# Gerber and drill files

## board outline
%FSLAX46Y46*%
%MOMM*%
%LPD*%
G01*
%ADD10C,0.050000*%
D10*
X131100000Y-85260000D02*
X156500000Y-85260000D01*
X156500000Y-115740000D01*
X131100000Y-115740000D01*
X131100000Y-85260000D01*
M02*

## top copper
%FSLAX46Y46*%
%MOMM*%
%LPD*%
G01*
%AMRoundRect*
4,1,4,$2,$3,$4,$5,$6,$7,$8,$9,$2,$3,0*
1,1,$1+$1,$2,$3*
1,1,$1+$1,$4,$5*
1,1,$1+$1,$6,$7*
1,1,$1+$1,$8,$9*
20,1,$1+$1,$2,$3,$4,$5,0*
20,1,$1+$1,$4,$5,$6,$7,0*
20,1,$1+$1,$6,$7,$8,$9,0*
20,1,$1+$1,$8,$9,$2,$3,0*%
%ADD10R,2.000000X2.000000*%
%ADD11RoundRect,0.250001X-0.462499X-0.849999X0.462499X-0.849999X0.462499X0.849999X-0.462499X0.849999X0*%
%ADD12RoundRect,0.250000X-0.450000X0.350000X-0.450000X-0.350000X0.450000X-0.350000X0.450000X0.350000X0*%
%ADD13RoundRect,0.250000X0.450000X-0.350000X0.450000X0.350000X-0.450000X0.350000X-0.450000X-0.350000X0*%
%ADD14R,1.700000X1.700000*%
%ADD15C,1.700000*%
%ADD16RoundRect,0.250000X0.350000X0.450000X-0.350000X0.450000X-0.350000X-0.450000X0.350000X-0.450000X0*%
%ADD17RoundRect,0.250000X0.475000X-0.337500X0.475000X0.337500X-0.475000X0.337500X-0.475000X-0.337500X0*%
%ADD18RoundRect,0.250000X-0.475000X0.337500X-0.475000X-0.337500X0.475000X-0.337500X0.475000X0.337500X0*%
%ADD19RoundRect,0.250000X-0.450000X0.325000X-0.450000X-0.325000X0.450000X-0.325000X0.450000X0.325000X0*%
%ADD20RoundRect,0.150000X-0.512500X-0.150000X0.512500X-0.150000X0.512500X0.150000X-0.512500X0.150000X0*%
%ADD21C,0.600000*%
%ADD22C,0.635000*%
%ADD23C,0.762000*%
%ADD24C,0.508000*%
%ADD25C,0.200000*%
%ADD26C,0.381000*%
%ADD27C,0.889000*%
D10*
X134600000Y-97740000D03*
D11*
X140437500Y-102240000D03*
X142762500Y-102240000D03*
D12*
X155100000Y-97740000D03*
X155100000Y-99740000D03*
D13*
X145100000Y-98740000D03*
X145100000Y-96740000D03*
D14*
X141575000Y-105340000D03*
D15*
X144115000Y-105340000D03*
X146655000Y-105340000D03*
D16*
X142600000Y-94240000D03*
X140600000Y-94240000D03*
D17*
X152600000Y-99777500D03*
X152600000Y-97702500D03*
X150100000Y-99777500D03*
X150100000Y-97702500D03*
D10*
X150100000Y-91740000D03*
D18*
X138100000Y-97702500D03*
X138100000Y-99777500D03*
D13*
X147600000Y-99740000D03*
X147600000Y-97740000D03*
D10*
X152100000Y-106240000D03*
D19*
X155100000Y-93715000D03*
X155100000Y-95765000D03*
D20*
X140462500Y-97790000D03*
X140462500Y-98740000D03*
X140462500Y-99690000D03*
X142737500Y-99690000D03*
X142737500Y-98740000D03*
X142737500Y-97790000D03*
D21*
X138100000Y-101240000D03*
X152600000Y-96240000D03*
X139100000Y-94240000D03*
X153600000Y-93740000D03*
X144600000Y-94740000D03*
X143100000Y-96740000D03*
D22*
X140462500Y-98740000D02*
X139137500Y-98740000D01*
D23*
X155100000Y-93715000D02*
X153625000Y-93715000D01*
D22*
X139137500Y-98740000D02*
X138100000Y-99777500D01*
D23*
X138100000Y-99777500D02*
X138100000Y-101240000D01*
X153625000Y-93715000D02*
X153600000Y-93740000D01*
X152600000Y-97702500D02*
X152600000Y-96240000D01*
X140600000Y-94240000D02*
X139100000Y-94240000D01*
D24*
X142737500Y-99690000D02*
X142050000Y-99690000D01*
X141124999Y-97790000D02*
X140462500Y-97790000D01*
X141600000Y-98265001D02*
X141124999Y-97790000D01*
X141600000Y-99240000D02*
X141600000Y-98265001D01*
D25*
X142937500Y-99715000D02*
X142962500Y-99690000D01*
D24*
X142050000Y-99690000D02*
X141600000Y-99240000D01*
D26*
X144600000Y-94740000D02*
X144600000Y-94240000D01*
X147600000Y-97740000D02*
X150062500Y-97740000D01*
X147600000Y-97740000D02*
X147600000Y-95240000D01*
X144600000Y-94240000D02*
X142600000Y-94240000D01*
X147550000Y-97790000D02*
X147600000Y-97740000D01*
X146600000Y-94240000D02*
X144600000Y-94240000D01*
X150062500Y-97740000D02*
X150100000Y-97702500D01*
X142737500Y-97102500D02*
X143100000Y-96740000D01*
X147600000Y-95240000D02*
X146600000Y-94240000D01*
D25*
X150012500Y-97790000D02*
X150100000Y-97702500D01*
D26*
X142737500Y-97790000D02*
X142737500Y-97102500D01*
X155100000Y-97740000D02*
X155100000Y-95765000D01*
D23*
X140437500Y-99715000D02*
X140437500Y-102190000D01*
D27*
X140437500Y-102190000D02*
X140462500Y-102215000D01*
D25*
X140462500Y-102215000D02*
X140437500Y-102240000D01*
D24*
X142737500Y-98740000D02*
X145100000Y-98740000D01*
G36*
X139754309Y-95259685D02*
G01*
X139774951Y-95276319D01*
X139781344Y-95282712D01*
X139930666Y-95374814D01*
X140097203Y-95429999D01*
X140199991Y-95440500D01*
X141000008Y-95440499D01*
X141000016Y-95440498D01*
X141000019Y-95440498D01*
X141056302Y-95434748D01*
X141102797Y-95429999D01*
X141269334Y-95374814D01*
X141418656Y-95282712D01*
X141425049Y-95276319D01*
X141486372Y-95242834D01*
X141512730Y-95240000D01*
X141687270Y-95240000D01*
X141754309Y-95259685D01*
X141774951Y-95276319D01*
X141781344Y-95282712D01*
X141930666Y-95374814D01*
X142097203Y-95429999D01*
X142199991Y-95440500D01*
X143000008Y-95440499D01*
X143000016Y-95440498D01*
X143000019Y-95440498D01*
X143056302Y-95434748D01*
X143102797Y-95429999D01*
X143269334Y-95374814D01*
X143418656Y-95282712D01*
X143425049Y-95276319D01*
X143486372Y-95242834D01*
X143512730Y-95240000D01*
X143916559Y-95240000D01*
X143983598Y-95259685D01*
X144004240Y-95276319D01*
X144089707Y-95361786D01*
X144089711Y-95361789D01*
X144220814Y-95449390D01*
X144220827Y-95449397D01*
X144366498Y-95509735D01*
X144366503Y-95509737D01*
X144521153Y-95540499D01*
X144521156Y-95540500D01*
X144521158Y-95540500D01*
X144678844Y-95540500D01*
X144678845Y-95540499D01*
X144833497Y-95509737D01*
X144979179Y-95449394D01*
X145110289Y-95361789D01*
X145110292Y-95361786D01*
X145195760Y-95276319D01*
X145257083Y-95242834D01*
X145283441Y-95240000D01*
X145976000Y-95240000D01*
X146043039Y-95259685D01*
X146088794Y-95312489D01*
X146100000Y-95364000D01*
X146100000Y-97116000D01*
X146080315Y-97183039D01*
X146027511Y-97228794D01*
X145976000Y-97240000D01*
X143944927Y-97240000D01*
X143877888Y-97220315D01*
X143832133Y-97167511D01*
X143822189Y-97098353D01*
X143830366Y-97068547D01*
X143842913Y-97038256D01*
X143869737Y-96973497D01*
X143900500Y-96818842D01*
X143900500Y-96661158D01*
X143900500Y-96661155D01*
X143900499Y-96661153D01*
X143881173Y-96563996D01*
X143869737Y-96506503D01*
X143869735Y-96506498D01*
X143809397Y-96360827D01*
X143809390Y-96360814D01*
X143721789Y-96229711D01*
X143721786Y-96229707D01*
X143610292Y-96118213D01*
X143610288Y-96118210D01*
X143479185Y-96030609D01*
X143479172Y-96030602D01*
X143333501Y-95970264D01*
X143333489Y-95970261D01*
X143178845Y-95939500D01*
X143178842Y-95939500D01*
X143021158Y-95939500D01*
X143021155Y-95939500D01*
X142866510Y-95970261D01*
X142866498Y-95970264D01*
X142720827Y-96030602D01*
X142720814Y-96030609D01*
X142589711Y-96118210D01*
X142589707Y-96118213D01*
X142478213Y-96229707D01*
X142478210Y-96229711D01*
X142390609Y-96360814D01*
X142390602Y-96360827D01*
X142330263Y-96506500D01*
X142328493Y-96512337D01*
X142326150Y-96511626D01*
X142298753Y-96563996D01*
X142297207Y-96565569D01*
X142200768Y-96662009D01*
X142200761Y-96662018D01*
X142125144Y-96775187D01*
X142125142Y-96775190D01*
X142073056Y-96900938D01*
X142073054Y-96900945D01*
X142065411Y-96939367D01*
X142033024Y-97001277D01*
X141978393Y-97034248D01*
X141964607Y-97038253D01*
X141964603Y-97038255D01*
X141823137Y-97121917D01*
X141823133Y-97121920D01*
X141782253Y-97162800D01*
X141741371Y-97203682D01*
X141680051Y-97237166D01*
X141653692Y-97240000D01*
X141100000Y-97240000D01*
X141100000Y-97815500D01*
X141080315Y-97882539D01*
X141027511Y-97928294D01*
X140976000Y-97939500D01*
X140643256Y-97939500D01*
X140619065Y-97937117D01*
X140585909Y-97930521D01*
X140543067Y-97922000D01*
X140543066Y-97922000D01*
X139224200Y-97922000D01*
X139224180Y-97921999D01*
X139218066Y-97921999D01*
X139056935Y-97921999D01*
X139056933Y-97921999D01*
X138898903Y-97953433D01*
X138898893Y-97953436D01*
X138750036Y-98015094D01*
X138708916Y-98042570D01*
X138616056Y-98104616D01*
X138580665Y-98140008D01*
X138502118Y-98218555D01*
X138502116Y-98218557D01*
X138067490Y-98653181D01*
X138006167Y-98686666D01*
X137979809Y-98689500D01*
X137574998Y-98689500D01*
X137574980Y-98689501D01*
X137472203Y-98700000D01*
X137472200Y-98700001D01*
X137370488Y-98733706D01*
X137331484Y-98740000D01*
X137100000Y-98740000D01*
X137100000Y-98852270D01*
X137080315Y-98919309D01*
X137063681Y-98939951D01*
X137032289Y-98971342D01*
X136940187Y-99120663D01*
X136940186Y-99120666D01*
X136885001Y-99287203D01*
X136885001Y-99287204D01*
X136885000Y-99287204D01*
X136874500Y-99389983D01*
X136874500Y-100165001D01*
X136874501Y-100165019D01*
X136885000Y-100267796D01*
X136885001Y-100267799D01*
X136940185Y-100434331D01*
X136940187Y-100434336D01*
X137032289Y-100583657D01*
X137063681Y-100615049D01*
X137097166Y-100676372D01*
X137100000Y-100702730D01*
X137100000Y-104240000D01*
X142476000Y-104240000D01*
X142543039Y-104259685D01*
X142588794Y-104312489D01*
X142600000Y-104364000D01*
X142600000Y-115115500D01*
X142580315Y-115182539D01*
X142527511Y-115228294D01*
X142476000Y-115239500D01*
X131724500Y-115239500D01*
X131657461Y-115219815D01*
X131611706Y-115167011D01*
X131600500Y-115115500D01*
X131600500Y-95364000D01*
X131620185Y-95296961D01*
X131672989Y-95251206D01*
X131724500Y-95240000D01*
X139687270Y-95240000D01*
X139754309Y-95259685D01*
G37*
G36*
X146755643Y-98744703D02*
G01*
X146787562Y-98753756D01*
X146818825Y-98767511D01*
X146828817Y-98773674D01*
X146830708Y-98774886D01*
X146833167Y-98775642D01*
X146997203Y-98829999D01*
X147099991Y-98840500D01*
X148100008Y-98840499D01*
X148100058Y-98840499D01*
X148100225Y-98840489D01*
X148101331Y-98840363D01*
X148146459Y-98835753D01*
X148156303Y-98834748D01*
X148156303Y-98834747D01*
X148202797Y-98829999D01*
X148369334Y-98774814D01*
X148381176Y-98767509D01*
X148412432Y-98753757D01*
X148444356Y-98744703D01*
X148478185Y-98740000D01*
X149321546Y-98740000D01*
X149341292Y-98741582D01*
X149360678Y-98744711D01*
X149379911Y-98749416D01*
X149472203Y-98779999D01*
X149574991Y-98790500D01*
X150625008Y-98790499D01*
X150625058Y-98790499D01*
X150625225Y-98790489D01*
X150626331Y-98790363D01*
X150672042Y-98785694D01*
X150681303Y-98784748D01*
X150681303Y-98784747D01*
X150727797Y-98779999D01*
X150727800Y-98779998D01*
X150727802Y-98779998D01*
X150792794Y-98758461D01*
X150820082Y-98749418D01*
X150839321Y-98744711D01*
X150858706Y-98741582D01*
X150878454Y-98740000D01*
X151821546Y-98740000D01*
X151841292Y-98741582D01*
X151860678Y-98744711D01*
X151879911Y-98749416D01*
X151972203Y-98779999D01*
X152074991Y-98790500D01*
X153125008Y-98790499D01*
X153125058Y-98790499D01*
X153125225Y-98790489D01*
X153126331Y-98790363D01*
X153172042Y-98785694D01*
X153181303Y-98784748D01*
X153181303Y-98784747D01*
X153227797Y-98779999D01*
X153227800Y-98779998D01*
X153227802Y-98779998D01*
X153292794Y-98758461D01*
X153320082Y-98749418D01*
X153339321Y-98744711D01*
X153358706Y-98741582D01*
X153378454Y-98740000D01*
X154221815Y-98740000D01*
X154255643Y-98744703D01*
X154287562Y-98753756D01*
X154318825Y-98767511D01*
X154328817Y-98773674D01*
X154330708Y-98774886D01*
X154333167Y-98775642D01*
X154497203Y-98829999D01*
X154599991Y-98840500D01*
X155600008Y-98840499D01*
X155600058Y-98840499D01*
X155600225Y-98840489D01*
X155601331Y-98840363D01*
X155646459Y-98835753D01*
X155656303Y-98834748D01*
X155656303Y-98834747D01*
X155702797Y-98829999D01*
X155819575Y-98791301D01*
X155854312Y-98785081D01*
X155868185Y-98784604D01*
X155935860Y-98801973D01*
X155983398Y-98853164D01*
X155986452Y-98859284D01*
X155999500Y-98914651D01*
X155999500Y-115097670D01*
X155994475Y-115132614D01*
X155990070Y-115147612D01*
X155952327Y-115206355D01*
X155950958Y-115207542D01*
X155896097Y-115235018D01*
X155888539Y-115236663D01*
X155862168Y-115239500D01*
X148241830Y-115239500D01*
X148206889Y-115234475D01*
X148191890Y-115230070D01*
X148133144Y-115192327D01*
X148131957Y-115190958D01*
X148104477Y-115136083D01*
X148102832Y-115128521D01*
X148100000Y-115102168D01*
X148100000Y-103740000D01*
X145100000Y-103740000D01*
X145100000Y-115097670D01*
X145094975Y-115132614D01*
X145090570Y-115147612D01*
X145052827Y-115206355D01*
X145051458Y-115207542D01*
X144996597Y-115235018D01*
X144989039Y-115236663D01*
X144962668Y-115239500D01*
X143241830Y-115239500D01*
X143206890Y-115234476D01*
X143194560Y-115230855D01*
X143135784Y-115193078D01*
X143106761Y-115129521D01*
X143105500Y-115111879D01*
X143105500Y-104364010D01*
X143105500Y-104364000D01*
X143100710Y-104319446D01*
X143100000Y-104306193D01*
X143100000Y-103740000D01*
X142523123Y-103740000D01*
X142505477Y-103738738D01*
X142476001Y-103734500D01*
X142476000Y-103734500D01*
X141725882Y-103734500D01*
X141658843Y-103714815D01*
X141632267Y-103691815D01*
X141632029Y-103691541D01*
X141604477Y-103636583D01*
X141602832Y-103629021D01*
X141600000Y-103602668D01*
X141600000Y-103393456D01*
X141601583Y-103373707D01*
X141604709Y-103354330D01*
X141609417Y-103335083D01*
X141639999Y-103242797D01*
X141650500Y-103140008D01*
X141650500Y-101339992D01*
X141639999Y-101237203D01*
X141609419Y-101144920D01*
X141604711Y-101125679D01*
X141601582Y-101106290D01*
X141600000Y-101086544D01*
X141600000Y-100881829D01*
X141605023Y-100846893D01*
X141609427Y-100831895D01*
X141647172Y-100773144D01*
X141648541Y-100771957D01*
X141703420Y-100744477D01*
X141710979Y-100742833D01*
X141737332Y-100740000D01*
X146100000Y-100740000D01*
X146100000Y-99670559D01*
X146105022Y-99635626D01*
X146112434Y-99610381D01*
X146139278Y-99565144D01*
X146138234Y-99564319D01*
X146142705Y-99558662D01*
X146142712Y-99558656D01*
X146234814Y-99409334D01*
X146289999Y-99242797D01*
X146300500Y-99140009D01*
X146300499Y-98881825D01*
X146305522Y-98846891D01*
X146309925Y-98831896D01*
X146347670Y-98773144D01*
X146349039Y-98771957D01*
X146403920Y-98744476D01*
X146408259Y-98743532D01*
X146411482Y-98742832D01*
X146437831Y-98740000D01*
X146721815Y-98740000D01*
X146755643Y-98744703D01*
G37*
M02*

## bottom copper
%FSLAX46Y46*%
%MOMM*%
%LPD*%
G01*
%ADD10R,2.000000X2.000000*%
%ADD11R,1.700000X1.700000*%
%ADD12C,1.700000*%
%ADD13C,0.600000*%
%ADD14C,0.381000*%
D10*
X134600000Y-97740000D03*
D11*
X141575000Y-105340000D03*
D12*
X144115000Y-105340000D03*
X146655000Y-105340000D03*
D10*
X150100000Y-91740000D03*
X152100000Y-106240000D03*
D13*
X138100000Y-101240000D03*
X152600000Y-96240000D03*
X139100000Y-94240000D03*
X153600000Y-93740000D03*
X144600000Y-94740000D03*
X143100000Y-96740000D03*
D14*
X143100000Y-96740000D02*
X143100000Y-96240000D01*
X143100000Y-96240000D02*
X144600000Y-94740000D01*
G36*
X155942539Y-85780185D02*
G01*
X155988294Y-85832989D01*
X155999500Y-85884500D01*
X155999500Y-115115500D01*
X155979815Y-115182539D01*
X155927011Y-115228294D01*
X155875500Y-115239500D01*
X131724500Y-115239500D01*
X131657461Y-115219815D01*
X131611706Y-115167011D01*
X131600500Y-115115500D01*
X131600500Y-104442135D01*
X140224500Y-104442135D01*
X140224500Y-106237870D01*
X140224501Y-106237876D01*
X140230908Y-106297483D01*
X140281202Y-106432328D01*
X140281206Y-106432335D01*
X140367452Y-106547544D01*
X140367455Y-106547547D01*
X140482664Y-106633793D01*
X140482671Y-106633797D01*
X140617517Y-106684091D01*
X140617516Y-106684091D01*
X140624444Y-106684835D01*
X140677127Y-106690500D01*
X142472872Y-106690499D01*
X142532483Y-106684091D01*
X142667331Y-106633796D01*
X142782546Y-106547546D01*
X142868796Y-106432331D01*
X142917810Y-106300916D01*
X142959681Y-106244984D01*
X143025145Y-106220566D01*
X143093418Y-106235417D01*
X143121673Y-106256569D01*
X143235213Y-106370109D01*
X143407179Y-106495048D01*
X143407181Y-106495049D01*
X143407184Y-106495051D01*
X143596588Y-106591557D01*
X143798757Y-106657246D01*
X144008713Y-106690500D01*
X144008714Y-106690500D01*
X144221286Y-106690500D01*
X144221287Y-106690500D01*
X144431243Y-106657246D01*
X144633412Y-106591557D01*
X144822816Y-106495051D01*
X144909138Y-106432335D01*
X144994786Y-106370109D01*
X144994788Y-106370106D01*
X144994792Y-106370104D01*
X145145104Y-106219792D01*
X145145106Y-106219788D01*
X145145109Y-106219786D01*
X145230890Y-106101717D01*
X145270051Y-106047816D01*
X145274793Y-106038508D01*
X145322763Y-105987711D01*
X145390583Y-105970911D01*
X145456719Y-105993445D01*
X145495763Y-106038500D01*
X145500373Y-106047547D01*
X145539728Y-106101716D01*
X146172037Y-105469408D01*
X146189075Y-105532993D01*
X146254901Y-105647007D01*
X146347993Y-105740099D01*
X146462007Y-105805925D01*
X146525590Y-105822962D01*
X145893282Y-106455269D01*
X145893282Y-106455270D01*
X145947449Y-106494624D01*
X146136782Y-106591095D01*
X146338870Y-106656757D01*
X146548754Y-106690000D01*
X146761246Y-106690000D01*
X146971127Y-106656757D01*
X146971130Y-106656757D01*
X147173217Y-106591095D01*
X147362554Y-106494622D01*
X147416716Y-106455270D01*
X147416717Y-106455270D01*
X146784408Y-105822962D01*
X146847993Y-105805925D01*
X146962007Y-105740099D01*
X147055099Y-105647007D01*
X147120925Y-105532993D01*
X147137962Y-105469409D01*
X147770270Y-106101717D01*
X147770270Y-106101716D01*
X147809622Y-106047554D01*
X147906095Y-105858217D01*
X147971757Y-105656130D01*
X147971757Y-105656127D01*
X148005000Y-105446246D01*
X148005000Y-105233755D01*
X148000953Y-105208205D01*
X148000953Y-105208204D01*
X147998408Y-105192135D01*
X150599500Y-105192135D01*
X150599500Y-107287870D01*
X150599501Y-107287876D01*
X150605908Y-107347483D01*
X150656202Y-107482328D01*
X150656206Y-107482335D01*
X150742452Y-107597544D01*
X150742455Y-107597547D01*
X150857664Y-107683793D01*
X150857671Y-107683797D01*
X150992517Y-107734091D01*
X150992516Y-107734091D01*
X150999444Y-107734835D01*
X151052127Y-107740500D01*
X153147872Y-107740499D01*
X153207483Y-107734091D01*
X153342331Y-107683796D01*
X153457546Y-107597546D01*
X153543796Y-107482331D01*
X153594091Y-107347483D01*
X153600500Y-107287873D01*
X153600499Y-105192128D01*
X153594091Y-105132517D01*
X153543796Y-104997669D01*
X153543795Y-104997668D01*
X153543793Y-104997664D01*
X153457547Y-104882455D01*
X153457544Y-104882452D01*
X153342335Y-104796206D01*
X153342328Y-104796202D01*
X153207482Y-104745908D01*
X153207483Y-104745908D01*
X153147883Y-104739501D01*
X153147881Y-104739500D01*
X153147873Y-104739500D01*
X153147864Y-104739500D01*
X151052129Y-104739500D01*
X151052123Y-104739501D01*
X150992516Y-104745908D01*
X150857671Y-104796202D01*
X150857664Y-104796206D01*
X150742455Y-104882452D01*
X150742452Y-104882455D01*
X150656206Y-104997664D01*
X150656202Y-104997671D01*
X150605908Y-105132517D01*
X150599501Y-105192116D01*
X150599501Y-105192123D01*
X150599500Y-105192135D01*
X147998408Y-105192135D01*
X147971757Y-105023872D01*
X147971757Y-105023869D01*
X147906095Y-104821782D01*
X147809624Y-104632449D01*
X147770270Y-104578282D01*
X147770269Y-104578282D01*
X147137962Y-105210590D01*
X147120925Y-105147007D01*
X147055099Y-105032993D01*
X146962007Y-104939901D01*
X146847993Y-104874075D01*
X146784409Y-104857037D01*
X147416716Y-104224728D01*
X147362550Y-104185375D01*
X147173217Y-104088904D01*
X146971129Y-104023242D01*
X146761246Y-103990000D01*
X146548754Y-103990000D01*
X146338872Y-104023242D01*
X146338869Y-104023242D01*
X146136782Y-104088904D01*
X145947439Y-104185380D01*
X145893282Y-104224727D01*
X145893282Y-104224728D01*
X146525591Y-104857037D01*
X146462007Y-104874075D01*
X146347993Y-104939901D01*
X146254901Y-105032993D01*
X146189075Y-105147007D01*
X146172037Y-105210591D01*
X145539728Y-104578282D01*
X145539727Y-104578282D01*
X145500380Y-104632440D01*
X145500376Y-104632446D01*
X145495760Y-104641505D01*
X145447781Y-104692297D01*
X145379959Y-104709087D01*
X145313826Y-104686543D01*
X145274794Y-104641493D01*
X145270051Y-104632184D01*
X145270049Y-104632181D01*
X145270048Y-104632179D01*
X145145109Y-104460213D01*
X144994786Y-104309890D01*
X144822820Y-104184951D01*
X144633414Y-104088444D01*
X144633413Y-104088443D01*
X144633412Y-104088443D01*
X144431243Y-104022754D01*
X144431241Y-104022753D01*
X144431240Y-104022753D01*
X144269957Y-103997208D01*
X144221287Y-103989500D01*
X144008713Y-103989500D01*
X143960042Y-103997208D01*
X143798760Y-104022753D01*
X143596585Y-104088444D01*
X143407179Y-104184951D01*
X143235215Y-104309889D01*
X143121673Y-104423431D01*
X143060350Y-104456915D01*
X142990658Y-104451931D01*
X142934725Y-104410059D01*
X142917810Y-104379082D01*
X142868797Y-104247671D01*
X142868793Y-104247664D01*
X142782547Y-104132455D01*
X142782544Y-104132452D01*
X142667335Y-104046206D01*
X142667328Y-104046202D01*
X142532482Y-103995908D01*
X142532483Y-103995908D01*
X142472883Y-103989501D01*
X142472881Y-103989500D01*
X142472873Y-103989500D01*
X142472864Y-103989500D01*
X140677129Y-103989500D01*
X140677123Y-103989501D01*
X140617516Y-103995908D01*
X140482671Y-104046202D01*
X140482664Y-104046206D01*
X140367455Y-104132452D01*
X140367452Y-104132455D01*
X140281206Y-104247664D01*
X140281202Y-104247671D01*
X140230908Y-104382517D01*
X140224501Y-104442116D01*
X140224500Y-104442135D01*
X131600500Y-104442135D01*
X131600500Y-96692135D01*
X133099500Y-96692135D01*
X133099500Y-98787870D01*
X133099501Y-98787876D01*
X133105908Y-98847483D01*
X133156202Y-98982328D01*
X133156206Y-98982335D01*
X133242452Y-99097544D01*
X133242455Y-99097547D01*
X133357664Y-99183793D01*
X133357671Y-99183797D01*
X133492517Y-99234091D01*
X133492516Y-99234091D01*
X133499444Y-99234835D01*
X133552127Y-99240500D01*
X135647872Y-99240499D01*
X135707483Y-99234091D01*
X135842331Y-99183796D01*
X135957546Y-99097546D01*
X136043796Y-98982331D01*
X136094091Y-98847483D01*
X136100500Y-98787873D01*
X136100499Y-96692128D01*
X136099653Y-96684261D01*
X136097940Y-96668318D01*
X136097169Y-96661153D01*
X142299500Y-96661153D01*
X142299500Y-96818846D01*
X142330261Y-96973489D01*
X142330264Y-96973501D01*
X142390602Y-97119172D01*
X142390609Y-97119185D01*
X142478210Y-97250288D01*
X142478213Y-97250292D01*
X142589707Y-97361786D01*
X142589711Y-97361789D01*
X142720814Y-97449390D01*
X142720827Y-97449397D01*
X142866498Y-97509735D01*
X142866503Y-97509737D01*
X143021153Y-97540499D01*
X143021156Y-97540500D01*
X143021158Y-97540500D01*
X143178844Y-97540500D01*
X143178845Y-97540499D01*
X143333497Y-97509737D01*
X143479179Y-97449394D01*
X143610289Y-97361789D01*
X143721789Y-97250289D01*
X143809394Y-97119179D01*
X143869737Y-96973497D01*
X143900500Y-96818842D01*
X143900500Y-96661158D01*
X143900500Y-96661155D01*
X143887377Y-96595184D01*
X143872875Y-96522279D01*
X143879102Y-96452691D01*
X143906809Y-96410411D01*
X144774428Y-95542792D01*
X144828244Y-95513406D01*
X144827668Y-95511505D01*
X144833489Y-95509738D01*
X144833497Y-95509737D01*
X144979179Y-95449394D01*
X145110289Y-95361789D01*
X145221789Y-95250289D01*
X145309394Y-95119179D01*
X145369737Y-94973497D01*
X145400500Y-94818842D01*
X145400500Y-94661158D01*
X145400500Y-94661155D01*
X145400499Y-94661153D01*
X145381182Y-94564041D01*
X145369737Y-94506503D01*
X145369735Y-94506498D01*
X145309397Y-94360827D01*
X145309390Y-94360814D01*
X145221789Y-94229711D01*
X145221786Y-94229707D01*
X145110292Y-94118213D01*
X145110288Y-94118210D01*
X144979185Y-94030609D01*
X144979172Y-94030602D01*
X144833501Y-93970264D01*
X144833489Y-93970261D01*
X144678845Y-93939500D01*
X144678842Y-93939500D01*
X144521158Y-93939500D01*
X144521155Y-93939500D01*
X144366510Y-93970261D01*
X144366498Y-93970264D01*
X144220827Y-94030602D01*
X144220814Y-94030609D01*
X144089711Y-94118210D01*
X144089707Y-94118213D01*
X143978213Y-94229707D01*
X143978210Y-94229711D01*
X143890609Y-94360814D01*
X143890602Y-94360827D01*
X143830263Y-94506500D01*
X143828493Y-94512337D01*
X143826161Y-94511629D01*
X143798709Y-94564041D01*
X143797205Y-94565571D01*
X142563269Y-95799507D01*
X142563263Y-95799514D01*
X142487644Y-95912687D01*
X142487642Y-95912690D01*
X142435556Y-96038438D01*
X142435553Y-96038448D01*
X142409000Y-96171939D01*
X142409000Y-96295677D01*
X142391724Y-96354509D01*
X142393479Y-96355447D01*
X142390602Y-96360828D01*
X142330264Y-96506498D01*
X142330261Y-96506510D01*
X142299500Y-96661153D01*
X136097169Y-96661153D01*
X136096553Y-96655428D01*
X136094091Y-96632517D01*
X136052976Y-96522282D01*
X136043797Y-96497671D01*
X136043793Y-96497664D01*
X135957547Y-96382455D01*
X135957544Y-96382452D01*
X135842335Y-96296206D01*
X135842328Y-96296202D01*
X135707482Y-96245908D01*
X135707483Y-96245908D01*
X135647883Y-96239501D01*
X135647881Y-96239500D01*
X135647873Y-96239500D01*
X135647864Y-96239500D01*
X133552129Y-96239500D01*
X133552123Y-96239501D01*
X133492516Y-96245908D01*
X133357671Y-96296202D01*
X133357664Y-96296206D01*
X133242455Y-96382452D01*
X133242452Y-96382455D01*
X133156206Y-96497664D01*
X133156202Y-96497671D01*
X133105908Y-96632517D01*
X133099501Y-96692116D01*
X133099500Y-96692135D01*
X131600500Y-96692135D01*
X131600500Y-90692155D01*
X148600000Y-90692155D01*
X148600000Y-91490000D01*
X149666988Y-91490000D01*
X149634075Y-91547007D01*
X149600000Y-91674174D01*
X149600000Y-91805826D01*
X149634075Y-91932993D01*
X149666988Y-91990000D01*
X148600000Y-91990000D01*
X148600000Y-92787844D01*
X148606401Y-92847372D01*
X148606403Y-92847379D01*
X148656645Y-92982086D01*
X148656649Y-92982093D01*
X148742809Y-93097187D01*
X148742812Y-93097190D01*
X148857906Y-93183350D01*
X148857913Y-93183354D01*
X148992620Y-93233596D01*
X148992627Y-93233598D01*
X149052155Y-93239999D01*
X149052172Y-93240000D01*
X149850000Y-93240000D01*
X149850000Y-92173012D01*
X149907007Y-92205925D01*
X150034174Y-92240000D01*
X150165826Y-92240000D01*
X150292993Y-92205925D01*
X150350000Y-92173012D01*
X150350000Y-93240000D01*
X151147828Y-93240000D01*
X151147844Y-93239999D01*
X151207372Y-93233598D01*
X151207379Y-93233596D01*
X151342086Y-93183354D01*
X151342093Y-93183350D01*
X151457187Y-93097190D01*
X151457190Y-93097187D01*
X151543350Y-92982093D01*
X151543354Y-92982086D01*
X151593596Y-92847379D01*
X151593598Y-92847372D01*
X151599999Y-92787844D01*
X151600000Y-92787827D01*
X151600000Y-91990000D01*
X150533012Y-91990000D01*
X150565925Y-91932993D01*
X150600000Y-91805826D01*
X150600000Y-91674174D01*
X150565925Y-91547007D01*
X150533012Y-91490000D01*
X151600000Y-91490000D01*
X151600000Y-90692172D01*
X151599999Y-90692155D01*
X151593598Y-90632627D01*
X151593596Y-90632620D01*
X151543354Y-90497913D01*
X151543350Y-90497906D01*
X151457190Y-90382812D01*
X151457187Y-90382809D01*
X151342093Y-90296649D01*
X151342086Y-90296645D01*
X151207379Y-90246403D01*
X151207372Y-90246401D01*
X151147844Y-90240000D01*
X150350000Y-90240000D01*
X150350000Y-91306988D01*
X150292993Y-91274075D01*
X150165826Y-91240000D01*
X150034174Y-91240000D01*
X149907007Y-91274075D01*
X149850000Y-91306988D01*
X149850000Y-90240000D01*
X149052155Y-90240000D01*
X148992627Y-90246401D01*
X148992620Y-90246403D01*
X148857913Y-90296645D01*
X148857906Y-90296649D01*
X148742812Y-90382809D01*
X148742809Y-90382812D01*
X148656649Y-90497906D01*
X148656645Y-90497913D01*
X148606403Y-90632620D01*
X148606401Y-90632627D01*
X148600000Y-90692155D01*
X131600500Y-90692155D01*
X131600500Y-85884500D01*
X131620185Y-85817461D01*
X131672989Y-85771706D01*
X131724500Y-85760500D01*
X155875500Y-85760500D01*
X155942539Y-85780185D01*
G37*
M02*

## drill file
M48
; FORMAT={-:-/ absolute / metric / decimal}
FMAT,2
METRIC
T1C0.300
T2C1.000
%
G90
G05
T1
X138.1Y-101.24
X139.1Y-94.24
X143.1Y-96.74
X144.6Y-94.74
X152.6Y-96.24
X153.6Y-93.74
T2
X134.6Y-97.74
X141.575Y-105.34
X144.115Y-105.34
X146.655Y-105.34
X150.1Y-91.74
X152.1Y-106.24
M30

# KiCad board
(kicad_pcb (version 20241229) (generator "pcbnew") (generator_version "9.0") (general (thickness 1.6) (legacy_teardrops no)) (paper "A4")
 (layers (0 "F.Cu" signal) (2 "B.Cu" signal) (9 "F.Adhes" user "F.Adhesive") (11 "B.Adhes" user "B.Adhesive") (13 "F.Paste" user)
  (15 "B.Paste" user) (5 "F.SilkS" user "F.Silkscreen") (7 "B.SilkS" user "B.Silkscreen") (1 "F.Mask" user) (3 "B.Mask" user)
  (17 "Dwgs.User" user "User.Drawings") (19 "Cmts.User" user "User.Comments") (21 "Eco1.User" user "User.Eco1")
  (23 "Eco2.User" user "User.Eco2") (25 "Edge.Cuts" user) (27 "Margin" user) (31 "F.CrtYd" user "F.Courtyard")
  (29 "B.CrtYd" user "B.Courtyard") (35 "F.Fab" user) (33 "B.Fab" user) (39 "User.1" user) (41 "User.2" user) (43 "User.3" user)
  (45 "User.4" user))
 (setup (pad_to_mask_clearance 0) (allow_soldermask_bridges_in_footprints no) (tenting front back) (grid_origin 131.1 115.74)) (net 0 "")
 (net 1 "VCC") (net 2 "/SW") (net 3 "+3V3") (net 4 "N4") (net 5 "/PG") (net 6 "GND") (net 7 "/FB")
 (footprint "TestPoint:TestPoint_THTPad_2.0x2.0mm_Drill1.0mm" (layer "F.Cu") (at 134.6 97.74)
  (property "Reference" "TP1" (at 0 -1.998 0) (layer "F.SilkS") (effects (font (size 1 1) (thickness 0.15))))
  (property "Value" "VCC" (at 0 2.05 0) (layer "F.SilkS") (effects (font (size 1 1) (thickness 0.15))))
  (pad "1" thru_hole rect (at 0 0) (size 2 2) (drill 1) (layers "*.Cu" "*.Mask") (remove_unused_layers no) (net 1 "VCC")))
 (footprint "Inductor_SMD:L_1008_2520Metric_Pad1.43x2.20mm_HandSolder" (layer "F.Cu") (at 141.6 102.24)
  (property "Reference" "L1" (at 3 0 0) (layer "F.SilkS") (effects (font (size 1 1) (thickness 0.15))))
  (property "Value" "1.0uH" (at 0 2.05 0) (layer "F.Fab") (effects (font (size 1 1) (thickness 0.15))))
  (pad "1" smd roundrect (at -1.1625 0) (size 1.425 2.2) (layers "F.Cu" "F.Mask" "F.Paste") (roundrect_rratio 0.175439) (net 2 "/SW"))
  (pad "2" smd roundrect (at 1.1625 0) (size 1.425 2.2) (layers "F.Cu" "F.Mask" "F.Paste") (roundrect_rratio 0.175439) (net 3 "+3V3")))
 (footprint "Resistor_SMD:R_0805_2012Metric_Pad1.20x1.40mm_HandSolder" (layer "F.Cu") (at 155.1 98.74 -90)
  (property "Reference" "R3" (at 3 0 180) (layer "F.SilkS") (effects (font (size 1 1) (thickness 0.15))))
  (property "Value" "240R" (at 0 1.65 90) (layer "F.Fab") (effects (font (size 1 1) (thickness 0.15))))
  (pad "1" smd roundrect (at -1 0 270) (size 1.2 1.4) (layers "F.Cu" "F.Mask" "F.Paste") (roundrect_rratio 0.208333) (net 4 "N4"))
  (pad "2" smd roundrect (at 1 0 270) (size 1.2 1.4) (layers "F.Cu" "F.Mask" "F.Paste") (roundrect_rratio 0.208333) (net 3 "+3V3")))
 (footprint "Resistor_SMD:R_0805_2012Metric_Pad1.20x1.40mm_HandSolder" (layer "F.Cu") (at 145.1 97.74 90)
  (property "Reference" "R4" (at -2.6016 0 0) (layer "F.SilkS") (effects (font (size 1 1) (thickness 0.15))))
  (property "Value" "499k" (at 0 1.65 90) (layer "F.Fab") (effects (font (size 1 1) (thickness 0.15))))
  (pad "1" smd roundrect (at -1 0 90) (size 1.2 1.4) (layers "F.Cu" "F.Mask" "F.Paste") (roundrect_rratio 0.208333) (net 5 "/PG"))
  (pad "2" smd roundrect (at 1 0 90) (size 1.2 1.4) (layers "F.Cu" "F.Mask" "F.Paste") (roundrect_rratio 0.208333) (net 1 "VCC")))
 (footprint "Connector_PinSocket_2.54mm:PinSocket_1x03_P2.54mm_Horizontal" (layer "F.Cu") (at 141.575 105.34 90)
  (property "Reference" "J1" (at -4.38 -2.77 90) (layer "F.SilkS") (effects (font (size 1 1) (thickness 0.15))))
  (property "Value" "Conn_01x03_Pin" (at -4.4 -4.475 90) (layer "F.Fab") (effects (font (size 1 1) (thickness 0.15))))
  (pad "1" thru_hole rect (at 0 0 90) (size 1.7 1.7) (drill 1) (layers "*.Cu" "*.Mask") (remove_unused_layers no) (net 1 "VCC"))
  (pad "2" thru_hole circle (at 0 2.54 90) (size 1.7 1.7) (drill 1) (layers "*.Cu" "*.Mask") (remove_unused_layers no) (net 3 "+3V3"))
  (pad "3" thru_hole circle (at 0 5.08 90) (size 1.7 1.7) (drill 1) (layers "*.Cu" "*.Mask") (remove_unused_layers no) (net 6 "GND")))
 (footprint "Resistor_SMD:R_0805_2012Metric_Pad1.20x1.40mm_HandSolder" (layer "F.Cu") (at 141.6 94.24 180)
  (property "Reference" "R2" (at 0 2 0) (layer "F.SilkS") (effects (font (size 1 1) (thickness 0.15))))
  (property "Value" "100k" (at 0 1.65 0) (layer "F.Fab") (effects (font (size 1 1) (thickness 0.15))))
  (pad "1" smd roundrect (at -1 0 180) (size 1.2 1.4) (layers "F.Cu" "F.Mask" "F.Paste") (roundrect_rratio 0.208333) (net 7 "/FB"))
  (pad "2" smd roundrect (at 1 0 180) (size 1.2 1.4) (layers "F.Cu" "F.Mask" "F.Paste") (roundrect_rratio 0.208333) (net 6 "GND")))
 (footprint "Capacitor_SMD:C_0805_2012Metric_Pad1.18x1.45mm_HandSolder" (layer "F.Cu") (at 152.6 98.74 90)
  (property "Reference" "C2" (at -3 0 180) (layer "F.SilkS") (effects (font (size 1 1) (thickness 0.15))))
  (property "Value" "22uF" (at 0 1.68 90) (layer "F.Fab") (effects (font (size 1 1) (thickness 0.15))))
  (pad "1" smd roundrect (at -1.0375 0 90) (size 1.175 1.45) (layers "F.Cu" "F.Mask" "F.Paste") (roundrect_rratio 0.212766) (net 3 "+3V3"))
  (pad "2" smd roundrect (at 1.0375 0 90) (size 1.175 1.45) (layers "F.Cu" "F.Mask" "F.Paste") (roundrect_rratio 0.212766) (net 6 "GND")))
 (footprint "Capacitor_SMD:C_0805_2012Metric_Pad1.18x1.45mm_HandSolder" (layer "F.Cu") (at 150.1 98.74 90)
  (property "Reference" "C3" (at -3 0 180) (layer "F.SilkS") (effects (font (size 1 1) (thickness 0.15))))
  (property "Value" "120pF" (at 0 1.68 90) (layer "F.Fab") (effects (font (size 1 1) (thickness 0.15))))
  (pad "1" smd roundrect (at -1.0375 0 90) (size 1.175 1.45) (layers "F.Cu" "F.Mask" "F.Paste") (roundrect_rratio 0.212766) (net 3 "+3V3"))
  (pad "2" smd roundrect (at 1.0375 0 90) (size 1.175 1.45) (layers "F.Cu" "F.Mask" "F.Paste") (roundrect_rratio 0.212766) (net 7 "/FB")))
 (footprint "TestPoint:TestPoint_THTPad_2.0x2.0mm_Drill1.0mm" (layer "F.Cu") (at 150.1 91.74)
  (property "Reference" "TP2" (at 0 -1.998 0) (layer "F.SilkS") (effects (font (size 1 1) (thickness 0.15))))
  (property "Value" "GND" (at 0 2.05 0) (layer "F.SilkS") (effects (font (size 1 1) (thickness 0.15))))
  (pad "1" thru_hole rect (at 0 0) (size 2 2) (drill 1) (layers "*.Cu" "*.Mask") (remove_unused_layers no) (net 6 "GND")))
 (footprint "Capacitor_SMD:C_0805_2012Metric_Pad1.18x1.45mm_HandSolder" (layer "F.Cu") (at 138.1 98.74 -90)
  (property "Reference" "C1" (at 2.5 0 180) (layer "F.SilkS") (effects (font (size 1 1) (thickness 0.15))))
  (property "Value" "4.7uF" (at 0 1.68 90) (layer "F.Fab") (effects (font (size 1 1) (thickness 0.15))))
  (pad "1" smd roundrect (at -1.0375 0 270) (size 1.175 1.45) (layers "F.Cu" "F.Mask" "F.Paste") (roundrect_rratio 0.212766) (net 1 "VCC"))
  (pad "2" smd roundrect (at 1.0375 0 270) (size 1.175 1.45) (layers "F.Cu" "F.Mask" "F.Paste") (roundrect_rratio 0.212766) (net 6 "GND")))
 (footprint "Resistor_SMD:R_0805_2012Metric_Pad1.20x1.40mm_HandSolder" (layer "F.Cu") (at 147.6 98.74 90)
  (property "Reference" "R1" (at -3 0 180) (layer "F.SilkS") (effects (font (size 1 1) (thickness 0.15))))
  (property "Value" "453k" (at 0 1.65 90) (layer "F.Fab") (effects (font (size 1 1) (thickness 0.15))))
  (pad "1" smd roundrect (at -1 0 90) (size 1.2 1.4) (layers "F.Cu" "F.Mask" "F.Paste") (roundrect_rratio 0.208333) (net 3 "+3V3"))
  (pad "2" smd roundrect (at 1 0 90) (size 1.2 1.4) (layers "F.Cu" "F.Mask" "F.Paste") (roundrect_rratio 0.208333) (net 7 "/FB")))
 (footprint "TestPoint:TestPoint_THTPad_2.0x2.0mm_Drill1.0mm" (layer "F.Cu") (at 152.1 106.24)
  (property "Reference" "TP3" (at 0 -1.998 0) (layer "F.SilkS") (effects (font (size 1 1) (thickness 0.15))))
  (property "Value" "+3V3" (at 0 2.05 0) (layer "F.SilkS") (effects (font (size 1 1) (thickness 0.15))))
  (pad "1" thru_hole rect (at 0 0) (size 2 2) (drill 1) (layers "*.Cu" "*.Mask") (remove_unused_layers no) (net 3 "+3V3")))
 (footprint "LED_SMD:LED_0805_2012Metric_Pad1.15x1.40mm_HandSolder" (layer "F.Cu") (at 155.1 94.74 -90)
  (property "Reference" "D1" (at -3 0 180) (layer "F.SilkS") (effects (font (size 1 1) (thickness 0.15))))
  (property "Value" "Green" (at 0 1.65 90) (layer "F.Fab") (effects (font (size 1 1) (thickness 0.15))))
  (pad "1" smd roundrect (at -1.025 0 270) (size 1.15 1.4) (layers "F.Cu" "F.Mask" "F.Paste") (roundrect_rratio 0.217391) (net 6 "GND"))
  (pad "2" smd roundrect (at 1.025 0 270) (size 1.15 1.4) (layers "F.Cu" "F.Mask" "F.Paste") (roundrect_rratio 0.217391) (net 4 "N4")))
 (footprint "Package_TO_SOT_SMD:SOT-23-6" (layer "F.Cu") (at 141.6 98.74)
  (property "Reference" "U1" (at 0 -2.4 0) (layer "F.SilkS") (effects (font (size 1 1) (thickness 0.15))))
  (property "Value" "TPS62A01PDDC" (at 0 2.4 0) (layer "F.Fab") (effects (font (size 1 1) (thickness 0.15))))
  (pad "1" smd roundrect (at -1.1375 -0.95) (size 1.325 0.6) (layers "F.Cu" "F.Mask" "F.Paste") (roundrect_rratio 0.25) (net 1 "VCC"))
  (pad "2" smd roundrect (at -1.1375 0) (size 1.325 0.6) (layers "F.Cu" "F.Mask" "F.Paste") (roundrect_rratio 0.25) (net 6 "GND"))
  (pad "3" smd roundrect (at -1.1375 0.95) (size 1.325 0.6) (layers "F.Cu" "F.Mask" "F.Paste") (roundrect_rratio 0.25) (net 2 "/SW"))
  (pad "4" smd roundrect (at 1.1375 0.95) (size 1.325 0.6) (layers "F.Cu" "F.Mask" "F.Paste") (roundrect_rratio 0.25) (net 1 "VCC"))
  (pad "5" smd roundrect (at 1.1375 0) (size 1.325 0.6) (layers "F.Cu" "F.Mask" "F.Paste") (roundrect_rratio 0.25) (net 5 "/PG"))
  (pad "6" smd roundrect (at 1.1375 -0.95) (size 1.325 0.6) (layers "F.Cu" "F.Mask" "F.Paste") (roundrect_rratio 0.25) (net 7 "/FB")))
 (gr_rect (start 131.1 85.26) (end 156.5 115.74) (stroke (width 0.05) (type default)) (fill no) (layer "Edge.Cuts"))
 (segment (start 140.4625 98.74) (end 139.1375 98.74) (width 0.635) (layer "F.Cu") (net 6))
 (segment (start 155.1 93.715) (end 153.625 93.715) (width 0.762) (layer "F.Cu") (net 6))
 (segment (start 139.1375 98.74) (end 138.1 99.7775) (width 0.635) (layer "F.Cu") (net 6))
 (segment (start 138.1 99.7775) (end 138.1 101.24) (width 0.762) (layer "F.Cu") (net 6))
 (segment (start 153.625 93.715) (end 153.6 93.74) (width 0.762) (layer "F.Cu") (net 6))
 (segment (start 152.6 97.7025) (end 152.6 96.24) (width 0.762) (layer "F.Cu") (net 6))
 (segment (start 140.6 94.24) (end 139.1 94.24) (width 0.762) (layer "F.Cu") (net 6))
 (via (at 138.1 101.24) (size 0.6) (drill 0.3) (layers "F.Cu" "B.Cu") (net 6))
 (via (at 152.6 96.24) (size 0.6) (drill 0.3) (layers "F.Cu" "B.Cu") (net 6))
 (via (at 139.1 94.24) (size 0.6) (drill 0.3) (layers "F.Cu" "B.Cu") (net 6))
 (via (at 153.6 93.74) (size 0.6) (drill 0.3) (layers "F.Cu" "B.Cu") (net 6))
 (segment (start 142.7375 99.69) (end 142.05 99.69) (width 0.508) (layer "F.Cu") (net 1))
 (segment (start 141.124999 97.79) (end 140.4625 97.79) (width 0.508) (layer "F.Cu") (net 1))
 (segment (start 141.6 98.265001) (end 141.124999 97.79) (width 0.508) (layer "F.Cu") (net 1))
 (segment (start 141.6 99.24) (end 141.6 98.265001) (width 0.508) (layer "F.Cu") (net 1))
 (segment (start 142.9375 99.715) (end 142.9625 99.69) (width 0.2) (layer "F.Cu") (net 1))
 (segment (start 142.05 99.69) (end 141.6 99.24) (width 0.508) (layer "F.Cu") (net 1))
 (segment (start 144.6 94.74) (end 144.6 94.24) (width 0.381) (layer "F.Cu") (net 7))
 (segment (start 147.6 97.74) (end 150.0625 97.74) (width 0.381) (layer "F.Cu") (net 7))
 (segment (start 147.6 97.74) (end 147.6 95.24) (width 0.381) (layer "F.Cu") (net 7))
 (segment (start 144.6 94.24) (end 142.6 94.24) (width 0.381) (layer "F.Cu") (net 7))
 (segment (start 147.55 97.79) (end 147.6 97.74) (width 0.381) (layer "F.Cu") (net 7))
 (segment (start 146.6 94.24) (end 144.6 94.24) (width 0.381) (layer "F.Cu") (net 7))
 (segment (start 150.0625 97.74) (end 150.1 97.7025) (width 0.381) (layer "F.Cu") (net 7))
 (segment (start 142.7375 97.1025) (end 143.1 96.74) (width 0.381) (layer "F.Cu") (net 7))
 (segment (start 147.6 95.24) (end 146.6 94.24) (width 0.381) (layer "F.Cu") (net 7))
 (segment (start 150.0125 97.79) (end 150.1 97.7025) (width 0.2) (layer "F.Cu") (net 7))
 (segment (start 142.7375 97.79) (end 142.7375 97.1025) (width 0.381) (layer "F.Cu") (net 7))
 (via (at 144.6 94.74) (size 0.6) (drill 0.3) (layers "F.Cu" "B.Cu") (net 7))
 (via (at 143.1 96.74) (size 0.6) (drill 0.3) (layers "F.Cu" "B.Cu") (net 7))
 (segment (start 143.1 96.74) (end 143.1 96.24) (width 0.381) (layer "B.Cu") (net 7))
 (segment (start 143.1 96.24) (end 144.6 94.74) (width 0.381) (layer "B.Cu") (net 7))
 (segment (start 155.1 97.74) (end 155.1 95.765) (width 0.381) (layer "F.Cu") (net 4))
 (segment (start 140.4375 99.715) (end 140.4375 102.19) (width 0.762) (layer "F.Cu") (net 2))
 (segment (start 140.4375 102.19) (end 140.4625 102.215) (width 0.889) (layer "F.Cu") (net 2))
 (segment (start 140.4625 102.215) (end 140.4375 102.24) (width 0.2) (layer "F.Cu") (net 2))
 (segment (start 142.7375 98.74) (end 145.1 98.74) (width 0.508) (layer "F.Cu") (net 5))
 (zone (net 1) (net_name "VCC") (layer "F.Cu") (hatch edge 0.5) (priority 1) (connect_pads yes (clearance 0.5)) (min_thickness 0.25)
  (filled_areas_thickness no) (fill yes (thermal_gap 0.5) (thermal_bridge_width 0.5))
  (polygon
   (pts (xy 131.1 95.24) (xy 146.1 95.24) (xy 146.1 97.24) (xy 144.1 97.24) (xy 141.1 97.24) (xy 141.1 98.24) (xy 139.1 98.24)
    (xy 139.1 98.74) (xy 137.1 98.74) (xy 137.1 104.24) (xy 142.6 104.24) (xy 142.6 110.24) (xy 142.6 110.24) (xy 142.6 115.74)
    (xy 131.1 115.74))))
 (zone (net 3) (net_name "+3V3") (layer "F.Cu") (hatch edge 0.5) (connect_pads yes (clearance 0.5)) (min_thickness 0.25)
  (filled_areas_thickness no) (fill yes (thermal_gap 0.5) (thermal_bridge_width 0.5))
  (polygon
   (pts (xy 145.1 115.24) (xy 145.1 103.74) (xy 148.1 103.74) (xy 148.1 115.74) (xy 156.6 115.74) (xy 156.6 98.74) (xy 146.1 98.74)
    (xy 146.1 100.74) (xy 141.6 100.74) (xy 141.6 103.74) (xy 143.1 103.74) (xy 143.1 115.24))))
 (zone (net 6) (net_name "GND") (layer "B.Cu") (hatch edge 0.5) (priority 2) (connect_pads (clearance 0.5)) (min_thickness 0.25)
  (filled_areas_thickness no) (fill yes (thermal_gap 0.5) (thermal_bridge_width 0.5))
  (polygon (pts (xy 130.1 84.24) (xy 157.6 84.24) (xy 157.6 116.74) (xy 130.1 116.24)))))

